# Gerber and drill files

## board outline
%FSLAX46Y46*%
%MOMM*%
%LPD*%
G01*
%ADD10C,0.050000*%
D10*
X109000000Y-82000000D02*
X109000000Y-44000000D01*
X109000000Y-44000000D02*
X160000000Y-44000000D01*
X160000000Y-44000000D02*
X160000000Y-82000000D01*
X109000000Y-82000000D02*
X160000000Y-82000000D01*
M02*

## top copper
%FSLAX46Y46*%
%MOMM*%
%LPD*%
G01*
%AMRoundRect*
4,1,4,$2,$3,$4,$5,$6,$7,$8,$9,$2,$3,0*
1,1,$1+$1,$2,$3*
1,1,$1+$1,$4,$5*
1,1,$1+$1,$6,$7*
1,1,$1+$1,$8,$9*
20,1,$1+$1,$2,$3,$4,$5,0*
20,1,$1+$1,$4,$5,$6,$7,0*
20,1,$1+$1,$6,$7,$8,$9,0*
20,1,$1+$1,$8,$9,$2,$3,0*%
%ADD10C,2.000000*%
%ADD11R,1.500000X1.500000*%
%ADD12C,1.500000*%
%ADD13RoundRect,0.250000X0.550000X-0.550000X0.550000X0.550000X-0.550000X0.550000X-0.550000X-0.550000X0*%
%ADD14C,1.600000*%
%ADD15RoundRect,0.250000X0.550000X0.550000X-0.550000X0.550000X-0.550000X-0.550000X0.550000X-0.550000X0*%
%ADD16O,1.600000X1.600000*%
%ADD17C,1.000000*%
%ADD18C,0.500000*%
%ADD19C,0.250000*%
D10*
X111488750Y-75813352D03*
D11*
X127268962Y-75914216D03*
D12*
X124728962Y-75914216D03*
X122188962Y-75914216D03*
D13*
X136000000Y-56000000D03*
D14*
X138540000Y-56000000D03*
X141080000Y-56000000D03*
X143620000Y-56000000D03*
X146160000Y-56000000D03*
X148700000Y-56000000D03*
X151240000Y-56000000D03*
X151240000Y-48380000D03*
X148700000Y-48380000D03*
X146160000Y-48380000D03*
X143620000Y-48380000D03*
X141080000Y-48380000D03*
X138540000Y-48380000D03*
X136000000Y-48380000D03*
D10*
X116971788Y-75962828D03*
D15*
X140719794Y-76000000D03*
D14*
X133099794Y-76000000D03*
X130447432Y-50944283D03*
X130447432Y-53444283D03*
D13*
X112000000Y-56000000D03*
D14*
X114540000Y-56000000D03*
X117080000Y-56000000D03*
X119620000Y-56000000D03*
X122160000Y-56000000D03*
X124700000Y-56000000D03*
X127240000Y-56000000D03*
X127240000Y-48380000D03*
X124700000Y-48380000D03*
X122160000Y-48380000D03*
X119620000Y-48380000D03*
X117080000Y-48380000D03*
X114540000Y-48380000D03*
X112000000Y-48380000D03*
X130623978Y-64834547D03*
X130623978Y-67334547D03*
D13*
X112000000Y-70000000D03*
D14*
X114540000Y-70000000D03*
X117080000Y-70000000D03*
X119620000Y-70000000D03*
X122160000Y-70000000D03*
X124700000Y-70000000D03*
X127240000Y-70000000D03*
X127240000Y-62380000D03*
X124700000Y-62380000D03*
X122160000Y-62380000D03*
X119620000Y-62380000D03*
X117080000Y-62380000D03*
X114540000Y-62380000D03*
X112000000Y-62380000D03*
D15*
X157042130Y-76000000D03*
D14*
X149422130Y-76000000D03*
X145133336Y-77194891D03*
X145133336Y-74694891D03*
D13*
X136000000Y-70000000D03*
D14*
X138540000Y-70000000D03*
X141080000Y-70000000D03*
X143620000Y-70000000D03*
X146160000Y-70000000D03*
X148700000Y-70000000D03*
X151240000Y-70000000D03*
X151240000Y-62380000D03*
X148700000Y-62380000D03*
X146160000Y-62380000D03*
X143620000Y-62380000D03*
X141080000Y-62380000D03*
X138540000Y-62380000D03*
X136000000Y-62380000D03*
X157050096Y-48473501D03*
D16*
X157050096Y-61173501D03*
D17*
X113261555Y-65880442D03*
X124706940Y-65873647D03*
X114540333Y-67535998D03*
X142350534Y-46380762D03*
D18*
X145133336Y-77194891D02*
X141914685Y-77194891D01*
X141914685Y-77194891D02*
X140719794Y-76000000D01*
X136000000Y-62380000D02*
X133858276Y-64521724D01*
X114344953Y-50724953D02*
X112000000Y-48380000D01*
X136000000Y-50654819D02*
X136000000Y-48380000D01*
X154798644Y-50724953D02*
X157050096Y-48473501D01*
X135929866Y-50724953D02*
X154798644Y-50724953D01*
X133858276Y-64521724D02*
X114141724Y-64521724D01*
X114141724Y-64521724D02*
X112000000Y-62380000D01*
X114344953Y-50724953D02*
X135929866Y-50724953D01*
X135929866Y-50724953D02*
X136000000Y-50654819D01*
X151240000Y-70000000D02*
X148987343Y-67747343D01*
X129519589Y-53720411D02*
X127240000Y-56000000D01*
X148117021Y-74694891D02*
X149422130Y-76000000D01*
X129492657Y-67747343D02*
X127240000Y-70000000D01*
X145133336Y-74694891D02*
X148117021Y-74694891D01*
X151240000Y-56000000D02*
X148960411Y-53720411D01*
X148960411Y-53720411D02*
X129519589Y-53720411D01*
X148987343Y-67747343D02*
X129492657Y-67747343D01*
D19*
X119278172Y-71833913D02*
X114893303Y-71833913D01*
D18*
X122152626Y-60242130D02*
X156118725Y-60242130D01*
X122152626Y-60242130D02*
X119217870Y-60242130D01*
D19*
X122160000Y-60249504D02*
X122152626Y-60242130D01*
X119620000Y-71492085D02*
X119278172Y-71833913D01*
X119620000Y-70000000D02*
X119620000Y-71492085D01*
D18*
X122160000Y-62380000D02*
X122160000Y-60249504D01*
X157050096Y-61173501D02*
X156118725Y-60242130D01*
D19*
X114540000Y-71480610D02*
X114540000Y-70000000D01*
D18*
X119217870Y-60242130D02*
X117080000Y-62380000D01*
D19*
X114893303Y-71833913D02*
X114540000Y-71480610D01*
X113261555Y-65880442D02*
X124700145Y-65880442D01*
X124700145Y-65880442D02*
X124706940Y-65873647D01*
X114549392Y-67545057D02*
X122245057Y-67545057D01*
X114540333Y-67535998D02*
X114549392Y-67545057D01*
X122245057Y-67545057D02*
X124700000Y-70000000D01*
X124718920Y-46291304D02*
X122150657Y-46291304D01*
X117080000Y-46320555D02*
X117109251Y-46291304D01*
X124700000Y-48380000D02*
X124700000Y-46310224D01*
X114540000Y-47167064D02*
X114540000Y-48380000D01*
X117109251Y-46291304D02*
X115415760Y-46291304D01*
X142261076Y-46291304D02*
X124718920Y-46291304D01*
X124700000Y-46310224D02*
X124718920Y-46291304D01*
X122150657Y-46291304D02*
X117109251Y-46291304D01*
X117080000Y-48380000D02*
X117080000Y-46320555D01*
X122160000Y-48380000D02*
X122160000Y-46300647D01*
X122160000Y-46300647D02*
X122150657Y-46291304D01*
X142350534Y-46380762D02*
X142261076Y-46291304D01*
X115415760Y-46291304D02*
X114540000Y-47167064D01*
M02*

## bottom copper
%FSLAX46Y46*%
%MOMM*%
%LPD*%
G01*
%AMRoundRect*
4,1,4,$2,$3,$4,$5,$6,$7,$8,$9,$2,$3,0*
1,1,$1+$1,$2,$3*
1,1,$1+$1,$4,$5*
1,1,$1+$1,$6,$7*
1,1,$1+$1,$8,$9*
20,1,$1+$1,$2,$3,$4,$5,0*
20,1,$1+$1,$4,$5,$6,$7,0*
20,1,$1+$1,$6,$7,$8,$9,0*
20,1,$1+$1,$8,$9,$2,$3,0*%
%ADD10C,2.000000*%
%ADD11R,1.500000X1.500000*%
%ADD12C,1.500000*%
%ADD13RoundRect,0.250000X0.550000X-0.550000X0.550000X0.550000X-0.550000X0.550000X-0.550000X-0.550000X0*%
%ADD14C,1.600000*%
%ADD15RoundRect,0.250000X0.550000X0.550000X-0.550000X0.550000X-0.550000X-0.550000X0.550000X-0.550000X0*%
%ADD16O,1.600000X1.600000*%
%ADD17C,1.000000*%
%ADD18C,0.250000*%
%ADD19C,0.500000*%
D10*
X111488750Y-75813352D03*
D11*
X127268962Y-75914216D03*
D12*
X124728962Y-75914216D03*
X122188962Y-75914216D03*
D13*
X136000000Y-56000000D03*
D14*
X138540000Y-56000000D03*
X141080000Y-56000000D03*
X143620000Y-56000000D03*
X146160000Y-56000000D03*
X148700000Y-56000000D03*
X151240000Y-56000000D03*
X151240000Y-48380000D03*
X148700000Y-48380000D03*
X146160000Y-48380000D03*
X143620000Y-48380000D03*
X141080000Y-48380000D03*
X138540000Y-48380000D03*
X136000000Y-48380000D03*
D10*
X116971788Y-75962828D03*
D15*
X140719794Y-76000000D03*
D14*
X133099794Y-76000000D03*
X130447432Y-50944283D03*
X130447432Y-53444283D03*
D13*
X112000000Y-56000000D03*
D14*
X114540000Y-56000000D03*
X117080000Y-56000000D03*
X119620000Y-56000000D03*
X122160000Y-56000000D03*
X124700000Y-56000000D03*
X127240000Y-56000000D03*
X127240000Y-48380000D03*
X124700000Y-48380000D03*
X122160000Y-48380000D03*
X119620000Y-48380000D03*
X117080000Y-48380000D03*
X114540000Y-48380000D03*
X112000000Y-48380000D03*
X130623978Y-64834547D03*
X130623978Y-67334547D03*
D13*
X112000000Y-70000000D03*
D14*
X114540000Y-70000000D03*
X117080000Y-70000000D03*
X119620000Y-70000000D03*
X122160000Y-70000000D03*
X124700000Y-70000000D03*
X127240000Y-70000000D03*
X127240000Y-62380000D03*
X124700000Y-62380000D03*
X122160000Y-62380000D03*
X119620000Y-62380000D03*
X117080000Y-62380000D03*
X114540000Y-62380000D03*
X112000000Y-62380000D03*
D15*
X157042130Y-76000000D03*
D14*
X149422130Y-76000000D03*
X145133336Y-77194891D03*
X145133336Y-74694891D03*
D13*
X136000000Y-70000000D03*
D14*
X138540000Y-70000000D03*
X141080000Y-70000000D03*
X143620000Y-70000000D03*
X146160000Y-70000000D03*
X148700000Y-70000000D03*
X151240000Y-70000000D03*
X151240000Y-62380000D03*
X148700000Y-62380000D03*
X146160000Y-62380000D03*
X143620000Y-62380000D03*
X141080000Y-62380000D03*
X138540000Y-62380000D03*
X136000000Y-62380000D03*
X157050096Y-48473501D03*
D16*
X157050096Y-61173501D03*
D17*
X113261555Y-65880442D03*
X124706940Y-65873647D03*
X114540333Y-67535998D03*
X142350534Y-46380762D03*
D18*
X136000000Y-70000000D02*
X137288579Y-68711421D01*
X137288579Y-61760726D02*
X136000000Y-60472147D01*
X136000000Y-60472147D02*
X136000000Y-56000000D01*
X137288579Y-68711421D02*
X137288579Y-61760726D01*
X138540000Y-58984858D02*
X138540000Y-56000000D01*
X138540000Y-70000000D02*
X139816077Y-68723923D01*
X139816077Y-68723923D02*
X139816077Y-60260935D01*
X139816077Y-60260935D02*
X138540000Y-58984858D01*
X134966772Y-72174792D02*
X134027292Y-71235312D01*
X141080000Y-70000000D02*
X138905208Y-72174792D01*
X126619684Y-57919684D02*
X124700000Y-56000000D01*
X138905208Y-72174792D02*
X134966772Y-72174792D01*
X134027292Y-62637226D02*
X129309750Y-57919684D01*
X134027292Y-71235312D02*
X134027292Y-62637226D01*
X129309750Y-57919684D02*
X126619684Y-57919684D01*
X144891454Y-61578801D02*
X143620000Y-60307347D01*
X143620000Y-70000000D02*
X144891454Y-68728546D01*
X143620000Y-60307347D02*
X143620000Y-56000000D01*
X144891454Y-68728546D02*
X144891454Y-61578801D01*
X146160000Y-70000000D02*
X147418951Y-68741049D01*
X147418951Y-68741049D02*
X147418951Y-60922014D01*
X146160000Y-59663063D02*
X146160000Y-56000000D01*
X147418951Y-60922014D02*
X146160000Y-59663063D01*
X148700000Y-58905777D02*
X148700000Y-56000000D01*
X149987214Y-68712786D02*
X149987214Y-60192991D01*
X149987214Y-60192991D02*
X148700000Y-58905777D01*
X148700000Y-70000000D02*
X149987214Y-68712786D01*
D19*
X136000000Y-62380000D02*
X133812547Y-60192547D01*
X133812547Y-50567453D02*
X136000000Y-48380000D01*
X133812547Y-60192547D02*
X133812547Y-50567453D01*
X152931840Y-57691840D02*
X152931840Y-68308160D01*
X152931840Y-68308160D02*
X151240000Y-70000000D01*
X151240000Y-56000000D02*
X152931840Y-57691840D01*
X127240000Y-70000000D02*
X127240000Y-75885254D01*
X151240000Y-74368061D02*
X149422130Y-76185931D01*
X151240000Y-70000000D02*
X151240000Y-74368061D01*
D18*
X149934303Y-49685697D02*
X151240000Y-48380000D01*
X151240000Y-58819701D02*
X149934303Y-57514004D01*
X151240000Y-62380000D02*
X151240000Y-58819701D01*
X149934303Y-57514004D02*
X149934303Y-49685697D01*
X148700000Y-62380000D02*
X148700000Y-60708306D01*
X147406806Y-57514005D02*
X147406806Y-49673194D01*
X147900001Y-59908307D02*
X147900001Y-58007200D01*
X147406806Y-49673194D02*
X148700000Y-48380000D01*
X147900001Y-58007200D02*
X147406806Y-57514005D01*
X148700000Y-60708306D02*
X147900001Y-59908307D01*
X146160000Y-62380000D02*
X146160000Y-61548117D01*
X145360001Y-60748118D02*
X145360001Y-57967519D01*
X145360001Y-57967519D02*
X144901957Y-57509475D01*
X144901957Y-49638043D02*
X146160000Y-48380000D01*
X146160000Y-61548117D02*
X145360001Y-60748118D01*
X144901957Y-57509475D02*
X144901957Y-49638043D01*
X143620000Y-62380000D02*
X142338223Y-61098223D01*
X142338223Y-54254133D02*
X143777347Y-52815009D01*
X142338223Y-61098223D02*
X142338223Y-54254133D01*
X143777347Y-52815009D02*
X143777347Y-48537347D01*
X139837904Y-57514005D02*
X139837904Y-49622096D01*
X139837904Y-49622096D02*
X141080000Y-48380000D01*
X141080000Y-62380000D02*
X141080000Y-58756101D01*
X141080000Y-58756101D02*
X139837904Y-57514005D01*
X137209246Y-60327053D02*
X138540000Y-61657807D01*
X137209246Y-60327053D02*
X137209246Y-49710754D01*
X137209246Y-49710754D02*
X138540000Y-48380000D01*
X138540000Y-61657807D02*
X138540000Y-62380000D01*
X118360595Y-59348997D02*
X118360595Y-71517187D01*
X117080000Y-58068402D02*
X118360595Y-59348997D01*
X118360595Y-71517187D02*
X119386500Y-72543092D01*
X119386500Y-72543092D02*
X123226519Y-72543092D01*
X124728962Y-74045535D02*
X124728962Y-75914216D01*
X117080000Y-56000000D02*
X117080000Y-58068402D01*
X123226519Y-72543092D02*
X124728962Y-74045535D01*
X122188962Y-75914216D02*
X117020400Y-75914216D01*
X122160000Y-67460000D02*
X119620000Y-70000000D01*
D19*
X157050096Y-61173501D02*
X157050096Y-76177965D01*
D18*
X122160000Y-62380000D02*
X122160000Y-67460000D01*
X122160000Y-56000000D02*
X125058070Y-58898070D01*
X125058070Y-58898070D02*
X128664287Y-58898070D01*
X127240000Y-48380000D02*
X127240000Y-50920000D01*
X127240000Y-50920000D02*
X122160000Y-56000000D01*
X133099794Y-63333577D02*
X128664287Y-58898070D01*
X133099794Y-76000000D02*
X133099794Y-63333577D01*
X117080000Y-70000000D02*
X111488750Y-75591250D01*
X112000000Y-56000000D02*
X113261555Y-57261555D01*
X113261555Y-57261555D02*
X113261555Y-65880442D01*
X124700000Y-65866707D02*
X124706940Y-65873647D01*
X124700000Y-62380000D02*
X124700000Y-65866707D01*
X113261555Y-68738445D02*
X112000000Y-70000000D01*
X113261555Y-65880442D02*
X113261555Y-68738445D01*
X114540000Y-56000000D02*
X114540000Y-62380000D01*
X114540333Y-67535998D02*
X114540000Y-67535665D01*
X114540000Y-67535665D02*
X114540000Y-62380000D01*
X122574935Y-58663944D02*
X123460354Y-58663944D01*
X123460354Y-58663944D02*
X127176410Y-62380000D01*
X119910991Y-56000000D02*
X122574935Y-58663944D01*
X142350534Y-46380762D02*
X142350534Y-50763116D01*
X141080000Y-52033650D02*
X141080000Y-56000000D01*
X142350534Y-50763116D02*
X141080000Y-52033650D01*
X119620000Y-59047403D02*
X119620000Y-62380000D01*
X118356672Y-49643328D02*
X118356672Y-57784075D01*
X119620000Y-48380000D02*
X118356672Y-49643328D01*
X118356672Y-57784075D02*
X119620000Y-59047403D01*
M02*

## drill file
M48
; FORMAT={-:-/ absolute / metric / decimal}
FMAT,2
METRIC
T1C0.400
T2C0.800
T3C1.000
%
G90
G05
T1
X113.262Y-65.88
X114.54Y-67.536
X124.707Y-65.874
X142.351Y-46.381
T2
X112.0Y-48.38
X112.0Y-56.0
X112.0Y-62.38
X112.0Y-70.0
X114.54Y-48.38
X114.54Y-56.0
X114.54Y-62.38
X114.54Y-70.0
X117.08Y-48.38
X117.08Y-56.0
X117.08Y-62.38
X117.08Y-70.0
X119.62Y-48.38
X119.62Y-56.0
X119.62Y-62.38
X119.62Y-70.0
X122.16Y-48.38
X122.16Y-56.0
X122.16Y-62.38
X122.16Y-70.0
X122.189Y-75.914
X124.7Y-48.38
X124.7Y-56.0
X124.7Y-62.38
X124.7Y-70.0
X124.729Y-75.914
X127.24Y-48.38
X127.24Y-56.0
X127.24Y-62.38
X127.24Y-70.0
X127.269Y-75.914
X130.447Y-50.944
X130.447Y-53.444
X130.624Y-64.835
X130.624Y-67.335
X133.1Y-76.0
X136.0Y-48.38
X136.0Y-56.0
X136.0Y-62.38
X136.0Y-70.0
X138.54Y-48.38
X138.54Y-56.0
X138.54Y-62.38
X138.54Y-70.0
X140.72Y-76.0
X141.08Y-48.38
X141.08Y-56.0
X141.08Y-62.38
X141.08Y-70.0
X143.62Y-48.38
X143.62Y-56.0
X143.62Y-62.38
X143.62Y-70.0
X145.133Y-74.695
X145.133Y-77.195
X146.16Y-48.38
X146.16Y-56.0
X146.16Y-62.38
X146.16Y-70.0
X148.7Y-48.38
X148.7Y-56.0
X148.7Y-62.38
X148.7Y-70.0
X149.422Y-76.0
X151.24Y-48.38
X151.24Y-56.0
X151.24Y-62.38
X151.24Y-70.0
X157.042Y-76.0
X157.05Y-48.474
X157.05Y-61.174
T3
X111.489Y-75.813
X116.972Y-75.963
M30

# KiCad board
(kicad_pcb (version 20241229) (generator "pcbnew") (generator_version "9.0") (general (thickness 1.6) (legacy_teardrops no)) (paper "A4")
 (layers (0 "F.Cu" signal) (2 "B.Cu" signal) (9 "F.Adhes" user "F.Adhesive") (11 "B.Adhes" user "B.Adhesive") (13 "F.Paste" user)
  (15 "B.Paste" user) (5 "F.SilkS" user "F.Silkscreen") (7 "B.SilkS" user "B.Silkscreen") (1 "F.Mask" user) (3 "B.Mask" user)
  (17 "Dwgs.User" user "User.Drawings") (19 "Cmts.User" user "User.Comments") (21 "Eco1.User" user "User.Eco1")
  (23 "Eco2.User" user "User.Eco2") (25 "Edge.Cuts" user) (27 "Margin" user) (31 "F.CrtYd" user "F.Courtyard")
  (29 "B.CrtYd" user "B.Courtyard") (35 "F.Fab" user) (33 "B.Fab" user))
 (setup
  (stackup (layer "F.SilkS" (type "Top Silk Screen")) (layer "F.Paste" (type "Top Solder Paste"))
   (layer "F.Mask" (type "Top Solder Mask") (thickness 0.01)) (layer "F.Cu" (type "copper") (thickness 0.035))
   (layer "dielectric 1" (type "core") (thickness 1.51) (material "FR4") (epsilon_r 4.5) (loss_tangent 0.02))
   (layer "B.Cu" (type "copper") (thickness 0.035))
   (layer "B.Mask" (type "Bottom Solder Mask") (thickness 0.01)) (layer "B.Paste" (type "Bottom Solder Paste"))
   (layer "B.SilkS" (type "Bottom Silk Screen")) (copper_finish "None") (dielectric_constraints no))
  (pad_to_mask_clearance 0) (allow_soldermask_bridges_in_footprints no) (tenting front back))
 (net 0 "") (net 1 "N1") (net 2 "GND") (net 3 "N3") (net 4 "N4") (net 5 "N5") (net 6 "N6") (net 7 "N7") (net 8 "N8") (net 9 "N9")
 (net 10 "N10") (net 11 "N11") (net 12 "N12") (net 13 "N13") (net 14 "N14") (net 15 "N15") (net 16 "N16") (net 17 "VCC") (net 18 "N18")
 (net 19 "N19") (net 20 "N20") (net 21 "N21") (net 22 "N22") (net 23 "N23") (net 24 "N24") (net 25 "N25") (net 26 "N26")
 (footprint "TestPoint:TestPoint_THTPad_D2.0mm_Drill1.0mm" (layer "F.Cu") (at 111.48875 75.813352)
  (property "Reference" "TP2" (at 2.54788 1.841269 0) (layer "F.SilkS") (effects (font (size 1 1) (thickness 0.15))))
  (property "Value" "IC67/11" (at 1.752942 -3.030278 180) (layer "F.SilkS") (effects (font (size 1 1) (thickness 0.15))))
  (pad "1" thru_hole circle (at 0 0) (size 2 2) (drill 1) (layers "*.Cu" "*.Mask") (remove_unused_layers no) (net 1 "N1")))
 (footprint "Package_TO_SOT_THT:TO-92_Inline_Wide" (layer "F.Cu") (at 127.268962 75.914216 180)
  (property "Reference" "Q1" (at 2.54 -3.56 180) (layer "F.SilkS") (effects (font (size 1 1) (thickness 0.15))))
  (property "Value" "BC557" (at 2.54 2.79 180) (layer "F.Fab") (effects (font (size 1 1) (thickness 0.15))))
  (pad "1" thru_hole rect (at 0 0 180) (size 1.5 1.5) (drill 0.8) (layers "*.Cu" "*.Mask") (remove_unused_layers no) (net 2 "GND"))
  (pad "2" thru_hole circle (at 2.54 0 180) (size 1.5 1.5) (drill 0.8) (layers "*.Cu" "*.Mask") (remove_unused_layers no) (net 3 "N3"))
  (pad "3" thru_hole circle (at 5.08 0 180) (size 1.5 1.5) (drill 0.8) (layers "*.Cu" "*.Mask") (remove_unused_layers no) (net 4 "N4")))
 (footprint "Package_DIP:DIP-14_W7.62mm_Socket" (layer "F.Cu") (at 136 56 90)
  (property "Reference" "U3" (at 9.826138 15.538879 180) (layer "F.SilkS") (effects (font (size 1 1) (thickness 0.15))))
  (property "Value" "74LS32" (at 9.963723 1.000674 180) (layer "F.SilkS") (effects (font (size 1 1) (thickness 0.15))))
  (pad "1" thru_hole roundrect (at 0 0 90) (size 1.6 1.6) (drill 0.8) (layers "*.Cu" "*.Mask") (remove_unused_layers no)
   (roundrect_rratio 0.15625) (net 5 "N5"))
  (pad "2" thru_hole circle (at 0 2.54 90) (size 1.6 1.6) (drill 0.8) (layers "*.Cu" "*.Mask") (remove_unused_layers no) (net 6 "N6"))
  (pad "3" thru_hole circle (at 0 5.08 90) (size 1.6 1.6) (drill 0.8) (layers "*.Cu" "*.Mask") (remove_unused_layers no) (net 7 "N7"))
  (pad "4" thru_hole circle (at 0 7.62 90) (size 1.6 1.6) (drill 0.8) (layers "*.Cu" "*.Mask") (remove_unused_layers no) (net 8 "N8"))
  (pad "5" thru_hole circle (at 0 10.16 90) (size 1.6 1.6) (drill 0.8) (layers "*.Cu" "*.Mask") (remove_unused_layers no) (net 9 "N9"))
  (pad "6" thru_hole circle (at 0 12.7 90) (size 1.6 1.6) (drill 0.8) (layers "*.Cu" "*.Mask") (remove_unused_layers no) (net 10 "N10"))
  (pad "7" thru_hole circle (at 0 15.24 90) (size 1.6 1.6) (drill 0.8) (layers "*.Cu" "*.Mask") (remove_unused_layers no) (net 2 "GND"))
  (pad "8" thru_hole circle (at 7.62 15.24 90) (size 1.6 1.6) (drill 0.8) (layers "*.Cu" "*.Mask") (remove_unused_layers no) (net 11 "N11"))
  (pad "9" thru_hole circle (at 7.62 12.7 90) (size 1.6 1.6) (drill 0.8) (layers "*.Cu" "*.Mask") (remove_unused_layers no) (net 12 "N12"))
  (pad "10" thru_hole circle (at 7.62 10.16 90) (size 1.6 1.6) (drill 0.8) (layers "*.Cu" "*.Mask") (remove_unused_layers no) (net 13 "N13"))
  (pad "11" thru_hole circle (at 7.62 7.62 90) (size 1.6 1.6) (drill 0.8) (layers "*.Cu" "*.Mask") (remove_unused_layers no) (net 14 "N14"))
  (pad "12" thru_hole circle (at 7.62 5.08 90) (size 1.6 1.6) (drill 0.8) (layers "*.Cu" "*.Mask") (remove_unused_layers no) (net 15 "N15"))
  (pad "13" thru_hole circle (at 7.62 2.54 90) (size 1.6 1.6) (drill 0.8) (layers "*.Cu" "*.Mask") (remove_unused_layers no) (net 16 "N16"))
  (pad "14" thru_hole circle (at 7.62 0 90) (size 1.6 1.6) (drill 0.8) (layers "*.Cu" "*.Mask") (remove_unused_layers no) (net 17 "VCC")))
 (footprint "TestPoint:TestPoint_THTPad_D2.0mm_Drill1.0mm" (layer "F.Cu") (at 116.971788 75.962828)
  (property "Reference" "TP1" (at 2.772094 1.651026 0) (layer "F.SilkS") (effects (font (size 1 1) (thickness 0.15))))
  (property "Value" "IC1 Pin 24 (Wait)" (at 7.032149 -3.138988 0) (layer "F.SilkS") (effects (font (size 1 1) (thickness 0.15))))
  (pad "1" thru_hole circle (at 0 0) (size 2 2) (drill 1) (layers "*.Cu" "*.Mask") (remove_unused_layers no) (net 4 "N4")))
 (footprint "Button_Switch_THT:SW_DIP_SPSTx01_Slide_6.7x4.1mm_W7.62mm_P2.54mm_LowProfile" (layer "F.Cu") (at 140.719794 76 180)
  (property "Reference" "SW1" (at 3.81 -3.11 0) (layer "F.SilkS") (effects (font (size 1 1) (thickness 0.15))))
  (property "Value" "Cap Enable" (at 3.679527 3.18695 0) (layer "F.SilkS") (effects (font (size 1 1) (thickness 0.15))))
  (pad "1" thru_hole roundrect (at 0 0 180) (size 1.6 1.6) (drill 0.8) (layers "*.Cu" "*.Mask") (remove_unused_layers no)
   (roundrect_rratio 0.15625) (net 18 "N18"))
  (pad "2" thru_hole circle (at 7.62 0 180) (size 1.6 1.6) (drill 0.8) (layers "*.Cu" "*.Mask") (remove_unused_layers no) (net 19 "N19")))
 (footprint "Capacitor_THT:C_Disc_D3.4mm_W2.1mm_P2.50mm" (layer "F.Cu") (at 130.447432 50.944283 -90)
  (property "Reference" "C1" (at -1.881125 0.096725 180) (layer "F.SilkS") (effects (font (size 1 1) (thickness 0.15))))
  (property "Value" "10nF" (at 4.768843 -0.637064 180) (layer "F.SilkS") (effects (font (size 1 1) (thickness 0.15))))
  (pad "1" thru_hole circle (at 0 0 270) (size 1.6 1.6) (drill 0.8) (layers "*.Cu" "*.Mask") (remove_unused_layers no) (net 17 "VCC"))
  (pad "2" thru_hole circle (at 2.5 0 270) (size 1.6 1.6) (drill 0.8) (layers "*.Cu" "*.Mask") (remove_unused_layers no) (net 2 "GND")))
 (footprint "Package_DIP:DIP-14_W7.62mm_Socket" (layer "F.Cu") (at 112 56 90)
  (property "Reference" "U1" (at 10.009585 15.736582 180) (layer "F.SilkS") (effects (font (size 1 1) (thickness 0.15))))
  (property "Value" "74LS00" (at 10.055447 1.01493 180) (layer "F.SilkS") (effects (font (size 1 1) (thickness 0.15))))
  (pad "1" thru_hole roundrect (at 0 0 90) (size 1.6 1.6) (drill 0.8) (layers "*.Cu" "*.Mask") (remove_unused_layers no)
   (roundrect_rratio 0.15625) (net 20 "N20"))
  (pad "2" thru_hole circle (at 0 2.54 90) (size 1.6 1.6) (drill 0.8) (layers "*.Cu" "*.Mask") (remove_unused_layers no) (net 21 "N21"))
  (pad "3" thru_hole circle (at 0 5.08 90) (size 1.6 1.6) (drill 0.8) (layers "*.Cu" "*.Mask") (remove_unused_layers no) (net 3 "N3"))
  (pad "4" thru_hole circle (at 0 7.62 90) (size 1.6 1.6) (drill 0.8) (layers "*.Cu" "*.Mask") (remove_unused_layers no) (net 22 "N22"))
  (pad "5" thru_hole circle (at 0 10.16 90) (size 1.6 1.6) (drill 0.8) (layers "*.Cu" "*.Mask") (remove_unused_layers no) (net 19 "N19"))
  (pad "6" thru_hole circle (at 0 12.7 90) (size 1.6 1.6) (drill 0.8) (layers "*.Cu" "*.Mask") (remove_unused_layers no) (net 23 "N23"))
  (pad "7" thru_hole circle (at 0 15.24 90) (size 1.6 1.6) (drill 0.8) (layers "*.Cu" "*.Mask") (remove_unused_layers no) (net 2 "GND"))
  (pad "8" thru_hole circle (at 7.62 15.24 90) (size 1.6 1.6) (drill 0.8) (layers "*.Cu" "*.Mask") (remove_unused_layers no) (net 19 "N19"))
  (pad "9" thru_hole circle (at 7.62 12.7 90) (size 1.6 1.6) (drill 0.8) (layers "*.Cu" "*.Mask") (remove_unused_layers no) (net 7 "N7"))
  (pad "10" thru_hole circle (at 7.62 10.16 90) (size 1.6 1.6) (drill 0.8) (layers "*.Cu" "*.Mask") (remove_unused_layers no) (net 7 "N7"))
  (pad "11" thru_hole circle (at 7.62 7.62 90) (size 1.6 1.6) (drill 0.8) (layers "*.Cu" "*.Mask") (remove_unused_layers no) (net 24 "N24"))
  (pad "12" thru_hole circle (at 7.62 5.08 90) (size 1.6 1.6) (drill 0.8) (layers "*.Cu" "*.Mask") (remove_unused_layers no) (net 7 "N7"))
  (pad "13" thru_hole circle (at 7.62 2.54 90) (size 1.6 1.6) (drill 0.8) (layers "*.Cu" "*.Mask") (remove_unused_layers no) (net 7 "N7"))
  (pad "14" thru_hole circle (at 7.62 0 90) (size 1.6 1.6) (drill 0.8) (layers "*.Cu" "*.Mask") (remove_unused_layers no) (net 17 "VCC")))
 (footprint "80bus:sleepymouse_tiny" (layer "F.Cu") (at 156.522194 67.890002)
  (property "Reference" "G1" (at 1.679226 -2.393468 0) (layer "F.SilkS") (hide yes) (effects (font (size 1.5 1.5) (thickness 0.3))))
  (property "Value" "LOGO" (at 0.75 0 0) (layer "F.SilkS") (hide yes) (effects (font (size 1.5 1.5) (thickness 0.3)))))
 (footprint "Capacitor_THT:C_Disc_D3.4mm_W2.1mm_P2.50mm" (layer "F.Cu") (at 130.623978 64.834547 -90)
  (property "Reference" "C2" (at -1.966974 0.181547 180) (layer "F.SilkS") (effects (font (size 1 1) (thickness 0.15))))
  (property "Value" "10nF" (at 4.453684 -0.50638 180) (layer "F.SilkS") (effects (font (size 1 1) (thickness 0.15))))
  (pad "1" thru_hole circle (at 0 0 270) (size 1.6 1.6) (drill 0.8) (layers "*.Cu" "*.Mask") (remove_unused_layers no) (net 17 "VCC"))
  (pad "2" thru_hole circle (at 2.5 0 270) (size 1.6 1.6) (drill 0.8) (layers "*.Cu" "*.Mask") (remove_unused_layers no) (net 2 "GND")))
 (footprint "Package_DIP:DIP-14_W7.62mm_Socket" (layer "F.Cu") (at 112 70 90)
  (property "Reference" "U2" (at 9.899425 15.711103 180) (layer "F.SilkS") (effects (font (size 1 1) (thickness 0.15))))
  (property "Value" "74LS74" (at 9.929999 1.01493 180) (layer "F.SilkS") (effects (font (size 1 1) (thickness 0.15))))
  (pad "1" thru_hole roundrect (at 0 0 90) (size 1.6 1.6) (drill 0.8) (layers "*.Cu" "*.Mask") (remove_unused_layers no)
   (roundrect_rratio 0.15625) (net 20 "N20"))
  (pad "2" thru_hole circle (at 0 2.54 90) (size 1.6 1.6) (drill 0.8) (layers "*.Cu" "*.Mask") (remove_unused_layers no) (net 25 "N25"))
  (pad "3" thru_hole circle (at 0 5.08 90) (size 1.6 1.6) (drill 0.8) (layers "*.Cu" "*.Mask") (remove_unused_layers no) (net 1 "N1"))
  (pad "4" thru_hole circle (at 0 7.62 90) (size 1.6 1.6) (drill 0.8) (layers "*.Cu" "*.Mask") (remove_unused_layers no) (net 25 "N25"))
  (pad "5" thru_hole circle (at 0 10.16 90) (size 1.6 1.6) (drill 0.8) (layers "*.Cu" "*.Mask") (remove_unused_layers no) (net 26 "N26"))
  (pad "6" thru_hole circle (at 0 12.7 90) (size 1.6 1.6) (drill 0.8) (layers "*.Cu" "*.Mask") (remove_unused_layers no) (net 21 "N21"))
  (pad "7" thru_hole circle (at 0 15.24 90) (size 1.6 1.6) (drill 0.8) (layers "*.Cu" "*.Mask") (remove_unused_layers no) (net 2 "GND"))
  (pad "8" thru_hole circle (at 7.62 15.24 90) (size 1.6 1.6) (drill 0.8) (layers "*.Cu" "*.Mask") (remove_unused_layers no) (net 22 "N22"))
  (pad "9" thru_hole circle (at 7.62 12.7 90) (size 1.6 1.6) (drill 0.8) (layers "*.Cu" "*.Mask") (remove_unused_layers no) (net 20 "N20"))
  (pad "10" thru_hole circle (at 7.62 10.16 90) (size 1.6 1.6) (drill 0.8) (layers "*.Cu" "*.Mask") (remove_unused_layers no) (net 25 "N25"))
  (pad "11" thru_hole circle (at 7.62 7.62 90) (size 1.6 1.6) (drill 0.8) (layers "*.Cu" "*.Mask") (remove_unused_layers no) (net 24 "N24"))
  (pad "12" thru_hole circle (at 7.62 5.08 90) (size 1.6 1.6) (drill 0.8) (layers "*.Cu" "*.Mask") (remove_unused_layers no) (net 25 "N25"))
  (pad "13" thru_hole circle (at 7.62 2.54 90) (size 1.6 1.6) (drill 0.8) (layers "*.Cu" "*.Mask") (remove_unused_layers no) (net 21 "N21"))
  (pad "14" thru_hole circle (at 7.62 0 90) (size 1.6 1.6) (drill 0.8) (layers "*.Cu" "*.Mask") (remove_unused_layers no) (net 17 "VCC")))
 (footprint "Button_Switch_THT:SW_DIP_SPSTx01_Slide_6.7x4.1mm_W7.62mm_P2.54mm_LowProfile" (layer "F.Cu") (at 157.04213 76 180)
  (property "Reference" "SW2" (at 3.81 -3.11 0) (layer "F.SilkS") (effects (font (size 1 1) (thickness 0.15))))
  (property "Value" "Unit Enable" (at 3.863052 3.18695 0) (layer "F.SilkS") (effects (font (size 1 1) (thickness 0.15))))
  (pad "1" thru_hole roundrect (at 0 0 180) (size 1.6 1.6) (drill 0.8) (layers "*.Cu" "*.Mask") (remove_unused_layers no)
   (roundrect_rratio 0.15625) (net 25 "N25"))
  (pad "2" thru_hole circle (at 7.62 0 180) (size 1.6 1.6) (drill 0.8) (layers "*.Cu" "*.Mask") (remove_unused_layers no) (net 2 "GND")))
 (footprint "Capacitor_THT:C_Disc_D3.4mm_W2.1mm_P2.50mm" (layer "F.Cu") (at 145.133336 77.194891 90)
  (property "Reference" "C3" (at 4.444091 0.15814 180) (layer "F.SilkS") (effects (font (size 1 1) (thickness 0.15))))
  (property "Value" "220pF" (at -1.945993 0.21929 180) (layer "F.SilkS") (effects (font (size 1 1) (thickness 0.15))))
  (pad "1" thru_hole circle (at 0 0 90) (size 1.6 1.6) (drill 0.8) (layers "*.Cu" "*.Mask") (remove_unused_layers no) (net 18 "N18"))
  (pad "2" thru_hole circle (at 2.5 0 90) (size 1.6 1.6) (drill 0.8) (layers "*.Cu" "*.Mask") (remove_unused_layers no) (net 2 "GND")))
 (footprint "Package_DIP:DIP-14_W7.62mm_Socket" (layer "F.Cu") (at 136 70 90)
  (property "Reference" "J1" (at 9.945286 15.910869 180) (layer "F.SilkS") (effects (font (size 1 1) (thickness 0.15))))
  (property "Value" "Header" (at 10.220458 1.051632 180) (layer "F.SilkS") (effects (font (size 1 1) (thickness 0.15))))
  (pad "1" thru_hole roundrect (at 0 0 90) (size 1.6 1.6) (drill 0.8) (layers "*.Cu" "*.Mask") (remove_unused_layers no)
   (roundrect_rratio 0.15625) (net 5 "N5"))
  (pad "2" thru_hole circle (at 0 2.54 90) (size 1.6 1.6) (drill 0.8) (layers "*.Cu" "*.Mask") (remove_unused_layers no) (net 6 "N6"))
  (pad "3" thru_hole circle (at 0 5.08 90) (size 1.6 1.6) (drill 0.8) (layers "*.Cu" "*.Mask") (remove_unused_layers no) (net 23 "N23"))
  (pad "4" thru_hole circle (at 0 7.62 90) (size 1.6 1.6) (drill 0.8) (layers "*.Cu" "*.Mask") (remove_unused_layers no) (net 8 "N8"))
  (pad "5" thru_hole circle (at 0 10.16 90) (size 1.6 1.6) (drill 0.8) (layers "*.Cu" "*.Mask") (remove_unused_layers no) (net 9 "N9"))
  (pad "6" thru_hole circle (at 0 12.7 90) (size 1.6 1.6) (drill 0.8) (layers "*.Cu" "*.Mask") (remove_unused_layers no) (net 10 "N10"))
  (pad "7" thru_hole circle (at 0 15.24 90) (size 1.6 1.6) (drill 0.8) (layers "*.Cu" "*.Mask") (remove_unused_layers no) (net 2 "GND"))
  (pad "8" thru_hole circle (at 7.62 15.24 90) (size 1.6 1.6) (drill 0.8) (layers "*.Cu" "*.Mask") (remove_unused_layers no) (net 11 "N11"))
  (pad "9" thru_hole circle (at 7.62 12.7 90) (size 1.6 1.6) (drill 0.8) (layers "*.Cu" "*.Mask") (remove_unused_layers no) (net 12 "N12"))
  (pad "10" thru_hole circle (at 7.62 10.16 90) (size 1.6 1.6) (drill 0.8) (layers "*.Cu" "*.Mask") (remove_unused_layers no) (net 13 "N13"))
  (pad "11" thru_hole circle (at 7.62 7.62 90) (size 1.6 1.6) (drill 0.8) (layers "*.Cu" "*.Mask") (remove_unused_layers no) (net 14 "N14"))
  (pad "12" thru_hole circle (at 7.62 5.08 90) (size 1.6 1.6) (drill 0.8) (layers "*.Cu" "*.Mask") (remove_unused_layers no) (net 15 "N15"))
  (pad "13" thru_hole circle (at 7.62 2.54 90) (size 1.6 1.6) (drill 0.8) (layers "*.Cu" "*.Mask") (remove_unused_layers no) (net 16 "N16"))
  (pad "14" thru_hole circle (at 7.62 0 90) (size 1.6 1.6) (drill 0.8) (layers "*.Cu" "*.Mask") (remove_unused_layers no) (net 17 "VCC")))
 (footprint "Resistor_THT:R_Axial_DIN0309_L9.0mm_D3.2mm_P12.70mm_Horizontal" (layer "F.Cu") (at 157.050096 48.473501 -90)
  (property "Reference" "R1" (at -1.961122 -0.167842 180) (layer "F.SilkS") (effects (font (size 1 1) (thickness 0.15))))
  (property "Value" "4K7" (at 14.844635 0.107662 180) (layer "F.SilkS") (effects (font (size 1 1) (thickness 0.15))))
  (pad "1" thru_hole circle (at 0 0 270) (size 1.6 1.6) (drill 0.8) (layers "*.Cu" "*.Mask") (remove_unused_layers no) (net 17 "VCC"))
  (pad "2" thru_hole oval (at 12.7 0 270) (size 1.6 1.6) (drill 0.8) (layers "*.Cu" "*.Mask") (remove_unused_layers no) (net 25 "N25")))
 (gr_line (start 109 82) (end 109 44) (stroke (width 0.05) (type solid)) (layer "Edge.Cuts"))
 (gr_line (start 109 44) (end 160 44) (stroke (width 0.05) (type solid)) (layer "Edge.Cuts"))
 (gr_line (start 160 44) (end 160 82) (stroke (width 0.05) (type solid)) (layer "Edge.Cuts"))
 (gr_line (start 109 82) (end 160 82) (stroke (width 0.05) (type solid)) (layer "Edge.Cuts"))
 (segment (start 145.133336 77.194891) (end 141.914685 77.194891) (width 0.5) (layer "F.Cu") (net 18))
 (segment (start 141.914685 77.194891) (end 140.719794 76) (width 0.5) (layer "F.Cu") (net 18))
 (segment (start 136 70) (end 137.288579 68.711421) (width 0.25) (layer "B.Cu") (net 5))
 (segment (start 137.288579 61.760726) (end 136 60.472147) (width 0.25) (layer "B.Cu") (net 5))
 (segment (start 136 60.472147) (end 136 56) (width 0.25) (layer "B.Cu") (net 5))
 (segment (start 137.288579 68.711421) (end 137.288579 61.760726) (width 0.25) (layer "B.Cu") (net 5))
 (segment (start 138.54 58.984858) (end 138.54 56) (width 0.25) (layer "B.Cu") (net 6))
 (segment (start 138.54 70) (end 139.816077 68.723923) (width 0.25) (layer "B.Cu") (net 6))
 (segment (start 139.816077 68.723923) (end 139.816077 60.260935) (width 0.25) (layer "B.Cu") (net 6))
 (segment (start 139.816077 60.260935) (end 138.54 58.984858) (width 0.25) (layer "B.Cu") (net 6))
 (segment (start 134.966772 72.174792) (end 134.027292 71.235312) (width 0.25) (layer "B.Cu") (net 23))
 (segment (start 141.08 70) (end 138.905208 72.174792) (width 0.25) (layer "B.Cu") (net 23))
 (segment (start 126.619684 57.919684) (end 124.7 56) (width 0.25) (layer "B.Cu") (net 23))
 (segment (start 138.905208 72.174792) (end 134.966772 72.174792) (width 0.25) (layer "B.Cu") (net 23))
 (segment (start 134.027292 62.637226) (end 129.30975 57.919684) (width 0.25) (layer "B.Cu") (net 23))
 (segment (start 134.027292 71.235312) (end 134.027292 62.637226) (width 0.25) (layer "B.Cu") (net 23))
 (segment (start 129.30975 57.919684) (end 126.619684 57.919684) (width 0.25) (layer "B.Cu") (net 23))
 (segment (start 144.891454 61.578801) (end 143.62 60.307347) (width 0.25) (layer "B.Cu") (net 8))
 (segment (start 143.62 70) (end 144.891454 68.728546) (width 0.25) (layer "B.Cu") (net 8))
 (segment (start 143.62 60.307347) (end 143.62 56) (width 0.25) (layer "B.Cu") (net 8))
 (segment (start 144.891454 68.728546) (end 144.891454 61.578801) (width 0.25) (layer "B.Cu") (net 8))
 (segment (start 146.16 70) (end 147.418951 68.741049) (width 0.25) (layer "B.Cu") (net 9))
 (segment (start 147.418951 68.741049) (end 147.418951 60.922014) (width 0.25) (layer "B.Cu") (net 9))
 (segment (start 146.16 59.663063) (end 146.16 56) (width 0.25) (layer "B.Cu") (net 9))
 (segment (start 147.418951 60.922014) (end 146.16 59.663063) (width 0.25) (layer "B.Cu") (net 9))
 (segment (start 148.7 58.905777) (end 148.7 56) (width 0.25) (layer "B.Cu") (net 10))
 (segment (start 149.987214 68.712786) (end 149.987214 60.192991) (width 0.25) (layer "B.Cu") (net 10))
 (segment (start 149.987214 60.192991) (end 148.7 58.905777) (width 0.25) (layer "B.Cu") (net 10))
 (segment (start 148.7 70) (end 149.987214 68.712786) (width 0.25) (layer "B.Cu") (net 10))
 (segment (start 136 62.38) (end 133.858276 64.521724) (width 0.5) (layer "F.Cu") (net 17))
 (segment (start 114.344953 50.724953) (end 112 48.38) (width 0.5) (layer "F.Cu") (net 17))
 (segment (start 136 50.654819) (end 136 48.38) (width 0.5) (layer "F.Cu") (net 17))
 (segment (start 154.798644 50.724953) (end 157.050096 48.473501) (width 0.5) (layer "F.Cu") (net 17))
 (segment (start 135.929866 50.724953) (end 154.798644 50.724953) (width 0.5) (layer "F.Cu") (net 17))
 (segment (start 133.858276 64.521724) (end 114.141724 64.521724) (width 0.5) (layer "F.Cu") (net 17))
 (segment (start 114.141724 64.521724) (end 112 62.38) (width 0.5) (layer "F.Cu") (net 17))
 (segment (start 114.344953 50.724953) (end 135.929866 50.724953) (width 0.5) (layer "F.Cu") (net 17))
 (segment (start 135.929866 50.724953) (end 136 50.654819) (width 0.5) (layer "F.Cu") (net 17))
 (segment (start 136 62.38) (end 133.812547 60.192547) (width 0.5) (layer "B.Cu") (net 17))
 (segment (start 133.812547 50.567453) (end 136 48.38) (width 0.5) (layer "B.Cu") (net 17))
 (segment (start 133.812547 60.192547) (end 133.812547 50.567453) (width 0.5) (layer "B.Cu") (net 17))
 (segment (start 151.24 70) (end 148.987343 67.747343) (width 0.5) (layer "F.Cu") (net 2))
 (segment (start 129.519589 53.720411) (end 127.24 56) (width 0.5) (layer "F.Cu") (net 2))
 (segment (start 148.117021 74.694891) (end 149.42213 76) (width 0.5) (layer "F.Cu") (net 2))
 (segment (start 129.492657 67.747343) (end 127.24 70) (width 0.5) (layer "F.Cu") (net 2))
 (segment (start 145.133336 74.694891) (end 148.117021 74.694891) (width 0.5) (layer "F.Cu") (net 2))
 (segment (start 151.24 56) (end 148.960411 53.720411) (width 0.5) (layer "F.Cu") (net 2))
 (segment (start 148.960411 53.720411) (end 129.519589 53.720411) (width 0.5) (layer "F.Cu") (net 2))
 (segment (start 148.987343 67.747343) (end 129.492657 67.747343) (width 0.5) (layer "F.Cu") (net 2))
 (segment (start 152.93184 57.69184) (end 152.93184 68.30816) (width 0.5) (layer "B.Cu") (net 2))
 (segment (start 152.93184 68.30816) (end 151.24 70) (width 0.5) (layer "B.Cu") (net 2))
 (segment (start 151.24 56) (end 152.93184 57.69184) (width 0.5) (layer "B.Cu") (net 2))
 (segment (start 127.24 70) (end 127.24 75.885254) (width 0.5) (layer "B.Cu") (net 2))
 (segment (start 151.24 74.368061) (end 149.42213 76.185931) (width 0.5) (layer "B.Cu") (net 2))
 (segment (start 151.24 70) (end 151.24 74.368061) (width 0.5) (layer "B.Cu") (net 2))
 (segment (start 149.934303 49.685697) (end 151.24 48.38) (width 0.25) (layer "B.Cu") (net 11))
 (segment (start 151.24 58.819701) (end 149.934303 57.514004) (width 0.25) (layer "B.Cu") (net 11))
 (segment (start 151.24 62.38) (end 151.24 58.819701) (width 0.25) (layer "B.Cu") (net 11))
 (segment (start 149.934303 57.514004) (end 149.934303 49.685697) (width 0.25) (layer "B.Cu") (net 11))
 (segment (start 148.7 62.38) (end 148.7 60.708306) (width 0.25) (layer "B.Cu") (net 12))
 (segment (start 147.406806 57.514005) (end 147.406806 49.673194) (width 0.25) (layer "B.Cu") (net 12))
 (segment (start 147.900001 59.908307) (end 147.900001 58.0072) (width 0.25) (layer "B.Cu") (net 12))
 (segment (start 147.406806 49.673194) (end 148.7 48.38) (width 0.25) (layer "B.Cu") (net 12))
 (segment (start 147.900001 58.0072) (end 147.406806 57.514005) (width 0.25) (layer "B.Cu") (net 12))
 (segment (start 148.7 60.708306) (end 147.900001 59.908307) (width 0.25) (layer "B.Cu") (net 12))
 (segment (start 146.16 62.38) (end 146.16 61.548117) (width 0.25) (layer "B.Cu") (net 13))
 (segment (start 145.360001 60.748118) (end 145.360001 57.967519) (width 0.25) (layer "B.Cu") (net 13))
 (segment (start 145.360001 57.967519) (end 144.901957 57.509475) (width 0.25) (layer "B.Cu") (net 13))
 (segment (start 144.901957 49.638043) (end 146.16 48.38) (width 0.25) (layer "B.Cu") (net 13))
 (segment (start 146.16 61.548117) (end 145.360001 60.748118) (width 0.25) (layer "B.Cu") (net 13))
 (segment (start 144.901957 57.509475) (end 144.901957 49.638043) (width 0.25) (layer "B.Cu") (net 13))
 (segment (start 143.62 62.38) (end 142.338223 61.098223) (width 0.25) (layer "B.Cu") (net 14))
 (segment (start 142.338223 54.254133) (end 143.777347 52.815009) (width 0.25) (layer "B.Cu") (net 14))
 (segment (start 142.338223 61.098223) (end 142.338223 54.254133) (width 0.25) (layer "B.Cu") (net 14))
 (segment (start 143.777347 52.815009) (end 143.777347 48.537347) (width 0.25) (layer "B.Cu") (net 14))
 (segment (start 139.837904 57.514005) (end 139.837904 49.622096) (width 0.25) (layer "B.Cu") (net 15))
 (segment (start 139.837904 49.622096) (end 141.08 48.38) (width 0.25) (layer "B.Cu") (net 15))
 (segment (start 141.08 62.38) (end 141.08 58.756101) (width 0.25) (layer "B.Cu") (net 15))
 (segment (start 141.08 58.756101) (end 139.837904 57.514005) (width 0.25) (layer "B.Cu") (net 15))
 (segment (start 137.209246 60.327053) (end 138.54 61.657807) (width 0.25) (layer "B.Cu") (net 16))
 (segment (start 137.209246 60.327053) (end 137.209246 49.710754) (width 0.25) (layer "B.Cu") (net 16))
 (segment (start 137.209246 49.710754) (end 138.54 48.38) (width 0.25) (layer "B.Cu") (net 16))
 (segment (start 138.54 61.657807) (end 138.54 62.38) (width 0.25) (layer "B.Cu") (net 16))
 (segment (start 118.360595 59.348997) (end 118.360595 71.517187) (width 0.25) (layer "B.Cu") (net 3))
 (segment (start 117.08 58.068402) (end 118.360595 59.348997) (width 0.25) (layer "B.Cu") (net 3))
 (segment (start 118.360595 71.517187) (end 119.3865 72.543092) (width 0.25) (layer "B.Cu") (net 3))
 (segment (start 119.3865 72.543092) (end 123.226519 72.543092) (width 0.25) (layer "B.Cu") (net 3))
 (segment (start 124.728962 74.045535) (end 124.728962 75.914216) (width 0.25) (layer "B.Cu") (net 3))
 (segment (start 117.08 56) (end 117.08 58.068402) (width 0.25) (layer "B.Cu") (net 3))
 (segment (start 123.226519 72.543092) (end 124.728962 74.045535) (width 0.25) (layer "B.Cu") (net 3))
 (segment (start 122.188962 75.914216) (end 117.0204 75.914216) (width 0.25) (layer "B.Cu") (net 4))
 (segment (start 119.278172 71.833913) (end 114.893303 71.833913) (width 0.25) (layer "F.Cu") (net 25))
 (segment (start 122.152626 60.24213) (end 156.118725 60.24213) (width 0.5) (layer "F.Cu") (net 25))
 (segment (start 122.152626 60.24213) (end 119.21787 60.24213) (width 0.5) (layer "F.Cu") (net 25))
 (segment (start 122.16 60.249504) (end 122.152626 60.24213) (width 0.25) (layer "F.Cu") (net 25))
 (segment (start 119.62 71.492085) (end 119.278172 71.833913) (width 0.25) (layer "F.Cu") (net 25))
 (segment (start 119.62 70) (end 119.62 71.492085) (width 0.25) (layer "F.Cu") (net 25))
 (segment (start 122.16 62.38) (end 122.16 60.249504) (width 0.5) (layer "F.Cu") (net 25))
 (segment (start 157.050096 61.173501) (end 156.118725 60.24213) (width 0.5) (layer "F.Cu") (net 25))
 (segment (start 114.54 71.48061) (end 114.54 70) (width 0.25) (layer "F.Cu") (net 25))
 (segment (start 119.21787 60.24213) (end 117.08 62.38) (width 0.5) (layer "F.Cu") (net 25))
 (segment (start 114.893303 71.833913) (end 114.54 71.48061) (width 0.25) (layer "F.Cu") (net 25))
 (segment (start 122.16 67.46) (end 119.62 70) (width 0.25) (layer "B.Cu") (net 25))
 (segment (start 157.050096 61.173501) (end 157.050096 76.177965) (width 0.5) (layer "B.Cu") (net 25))
 (segment (start 122.16 62.38) (end 122.16 67.46) (width 0.25) (layer "B.Cu") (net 25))
 (segment (start 122.16 56) (end 125.05807 58.89807) (width 0.25) (layer "B.Cu") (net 19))
 (segment (start 125.05807 58.89807) (end 128.664287 58.89807) (width 0.25) (layer "B.Cu") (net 19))
 (segment (start 127.24 48.38) (end 127.24 50.92) (width 0.25) (layer "B.Cu") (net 19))
 (segment (start 127.24 50.92) (end 122.16 56) (width 0.25) (layer "B.Cu") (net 19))
 (segment (start 133.099794 63.333577) (end 128.664287 58.89807) (width 0.25) (layer "B.Cu") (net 19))
 (segment (start 133.099794 76) (end 133.099794 63.333577) (width 0.25) (layer "B.Cu") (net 19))
 (segment (start 117.08 70) (end 111.48875 75.59125) (width 0.25) (layer "B.Cu") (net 1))
 (segment (start 113.261555 65.880442) (end 124.700145 65.880442) (width 0.25) (layer "F.Cu") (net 20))
 (segment (start 124.700145 65.880442) (end 124.70694 65.873647) (width 0.25) (layer "F.Cu") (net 20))
 (via (at 113.261555 65.880442) (size 1) (drill 0.4) (layers "F.Cu" "B.Cu") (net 20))
 (via (at 124.70694 65.873647) (size 1) (drill 0.4) (layers "F.Cu" "B.Cu") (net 20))
 (segment (start 112 56) (end 113.261555 57.261555) (width 0.25) (layer "B.Cu") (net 20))
 (segment (start 113.261555 57.261555) (end 113.261555 65.880442) (width 0.25) (layer "B.Cu") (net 20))
 (segment (start 124.7 65.866707) (end 124.70694 65.873647) (width 0.25) (layer "B.Cu") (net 20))
 (segment (start 124.7 62.38) (end 124.7 65.866707) (width 0.25) (layer "B.Cu") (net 20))
 (segment (start 113.261555 68.738445) (end 112 70) (width 0.25) (layer "B.Cu") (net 20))
 (segment (start 113.261555 65.880442) (end 113.261555 68.738445) (width 0.25) (layer "B.Cu") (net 20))
 (segment (start 114.549392 67.545057) (end 122.245057 67.545057) (width 0.25) (layer "F.Cu") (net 21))
 (segment (start 114.540333 67.535998) (end 114.549392 67.545057) (width 0.25) (layer "F.Cu") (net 21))
 (segment (start 122.245057 67.545057) (end 124.7 70) (width 0.25) (layer "F.Cu") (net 21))
 (via (at 114.540333 67.535998) (size 1) (drill 0.4) (layers "F.Cu" "B.Cu") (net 21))
 (segment (start 114.54 56) (end 114.54 62.38) (width 0.25) (layer "B.Cu") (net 21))
 (segment (start 114.540333 67.535998) (end 114.54 67.535665) (width 0.25) (layer "B.Cu") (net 21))
 (segment (start 114.54 67.535665) (end 114.54 62.38) (width 0.25) (layer "B.Cu") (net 21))
 (segment (start 122.574935 58.663944) (end 123.460354 58.663944) (width 0.25) (layer "B.Cu") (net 22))
 (segment (start 123.460354 58.663944) (end 127.17641 62.38) (width 0.25) (layer "B.Cu") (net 22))
 (segment (start 119.910991 56) (end 122.574935 58.663944) (width 0.25) (layer "B.Cu") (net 22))
 (segment (start 124.71892 46.291304) (end 122.150657 46.291304) (width 0.25) (layer "F.Cu") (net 7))
 (segment (start 117.08 46.320555) (end 117.109251 46.291304) (width 0.25) (layer "F.Cu") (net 7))
 (segment (start 124.7 48.38) (end 124.7 46.310224) (width 0.25) (layer "F.Cu") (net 7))
 (segment (start 114.54 47.167064) (end 114.54 48.38) (width 0.25) (layer "F.Cu") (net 7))
 (segment (start 117.109251 46.291304) (end 115.41576 46.291304) (width 0.25) (layer "F.Cu") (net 7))
 (segment (start 142.261076 46.291304) (end 124.71892 46.291304) (width 0.25) (layer "F.Cu") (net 7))
 (segment (start 124.7 46.310224) (end 124.71892 46.291304) (width 0.25) (layer "F.Cu") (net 7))
 (segment (start 122.150657 46.291304) (end 117.109251 46.291304) (width 0.25) (layer "F.Cu") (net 7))
 (segment (start 117.08 48.38) (end 117.08 46.320555) (width 0.25) (layer "F.Cu") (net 7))
 (segment (start 122.16 48.38) (end 122.16 46.300647) (width 0.25) (layer "F.Cu") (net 7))
 (segment (start 122.16 46.300647) (end 122.150657 46.291304) (width 0.25) (layer "F.Cu") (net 7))
 (segment (start 142.350534 46.380762) (end 142.261076 46.291304) (width 0.25) (layer "F.Cu") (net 7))
 (segment (start 115.41576 46.291304) (end 114.54 47.167064) (width 0.25) (layer "F.Cu") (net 7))
 (via (at 142.350534 46.380762) (size 1) (drill 0.4) (layers "F.Cu" "B.Cu") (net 7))
 (segment (start 142.350534 46.380762) (end 142.350534 50.763116) (width 0.25) (layer "B.Cu") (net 7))
 (segment (start 141.08 52.03365) (end 141.08 56) (width 0.25) (layer "B.Cu") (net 7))
 (segment (start 142.350534 50.763116) (end 141.08 52.03365) (width 0.25) (layer "B.Cu") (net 7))
 (segment (start 119.62 59.047403) (end 119.62 62.38) (width 0.25) (layer "B.Cu") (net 24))
 (segment (start 118.356672 49.643328) (end 118.356672 57.784075) (width 0.25) (layer "B.Cu") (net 24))
 (segment (start 119.62 48.38) (end 118.356672 49.643328) (width 0.25) (layer "B.Cu") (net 24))
 (segment (start 118.356672 57.784075) (end 119.62 59.047403) (width 0.25) (layer "B.Cu") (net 24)))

